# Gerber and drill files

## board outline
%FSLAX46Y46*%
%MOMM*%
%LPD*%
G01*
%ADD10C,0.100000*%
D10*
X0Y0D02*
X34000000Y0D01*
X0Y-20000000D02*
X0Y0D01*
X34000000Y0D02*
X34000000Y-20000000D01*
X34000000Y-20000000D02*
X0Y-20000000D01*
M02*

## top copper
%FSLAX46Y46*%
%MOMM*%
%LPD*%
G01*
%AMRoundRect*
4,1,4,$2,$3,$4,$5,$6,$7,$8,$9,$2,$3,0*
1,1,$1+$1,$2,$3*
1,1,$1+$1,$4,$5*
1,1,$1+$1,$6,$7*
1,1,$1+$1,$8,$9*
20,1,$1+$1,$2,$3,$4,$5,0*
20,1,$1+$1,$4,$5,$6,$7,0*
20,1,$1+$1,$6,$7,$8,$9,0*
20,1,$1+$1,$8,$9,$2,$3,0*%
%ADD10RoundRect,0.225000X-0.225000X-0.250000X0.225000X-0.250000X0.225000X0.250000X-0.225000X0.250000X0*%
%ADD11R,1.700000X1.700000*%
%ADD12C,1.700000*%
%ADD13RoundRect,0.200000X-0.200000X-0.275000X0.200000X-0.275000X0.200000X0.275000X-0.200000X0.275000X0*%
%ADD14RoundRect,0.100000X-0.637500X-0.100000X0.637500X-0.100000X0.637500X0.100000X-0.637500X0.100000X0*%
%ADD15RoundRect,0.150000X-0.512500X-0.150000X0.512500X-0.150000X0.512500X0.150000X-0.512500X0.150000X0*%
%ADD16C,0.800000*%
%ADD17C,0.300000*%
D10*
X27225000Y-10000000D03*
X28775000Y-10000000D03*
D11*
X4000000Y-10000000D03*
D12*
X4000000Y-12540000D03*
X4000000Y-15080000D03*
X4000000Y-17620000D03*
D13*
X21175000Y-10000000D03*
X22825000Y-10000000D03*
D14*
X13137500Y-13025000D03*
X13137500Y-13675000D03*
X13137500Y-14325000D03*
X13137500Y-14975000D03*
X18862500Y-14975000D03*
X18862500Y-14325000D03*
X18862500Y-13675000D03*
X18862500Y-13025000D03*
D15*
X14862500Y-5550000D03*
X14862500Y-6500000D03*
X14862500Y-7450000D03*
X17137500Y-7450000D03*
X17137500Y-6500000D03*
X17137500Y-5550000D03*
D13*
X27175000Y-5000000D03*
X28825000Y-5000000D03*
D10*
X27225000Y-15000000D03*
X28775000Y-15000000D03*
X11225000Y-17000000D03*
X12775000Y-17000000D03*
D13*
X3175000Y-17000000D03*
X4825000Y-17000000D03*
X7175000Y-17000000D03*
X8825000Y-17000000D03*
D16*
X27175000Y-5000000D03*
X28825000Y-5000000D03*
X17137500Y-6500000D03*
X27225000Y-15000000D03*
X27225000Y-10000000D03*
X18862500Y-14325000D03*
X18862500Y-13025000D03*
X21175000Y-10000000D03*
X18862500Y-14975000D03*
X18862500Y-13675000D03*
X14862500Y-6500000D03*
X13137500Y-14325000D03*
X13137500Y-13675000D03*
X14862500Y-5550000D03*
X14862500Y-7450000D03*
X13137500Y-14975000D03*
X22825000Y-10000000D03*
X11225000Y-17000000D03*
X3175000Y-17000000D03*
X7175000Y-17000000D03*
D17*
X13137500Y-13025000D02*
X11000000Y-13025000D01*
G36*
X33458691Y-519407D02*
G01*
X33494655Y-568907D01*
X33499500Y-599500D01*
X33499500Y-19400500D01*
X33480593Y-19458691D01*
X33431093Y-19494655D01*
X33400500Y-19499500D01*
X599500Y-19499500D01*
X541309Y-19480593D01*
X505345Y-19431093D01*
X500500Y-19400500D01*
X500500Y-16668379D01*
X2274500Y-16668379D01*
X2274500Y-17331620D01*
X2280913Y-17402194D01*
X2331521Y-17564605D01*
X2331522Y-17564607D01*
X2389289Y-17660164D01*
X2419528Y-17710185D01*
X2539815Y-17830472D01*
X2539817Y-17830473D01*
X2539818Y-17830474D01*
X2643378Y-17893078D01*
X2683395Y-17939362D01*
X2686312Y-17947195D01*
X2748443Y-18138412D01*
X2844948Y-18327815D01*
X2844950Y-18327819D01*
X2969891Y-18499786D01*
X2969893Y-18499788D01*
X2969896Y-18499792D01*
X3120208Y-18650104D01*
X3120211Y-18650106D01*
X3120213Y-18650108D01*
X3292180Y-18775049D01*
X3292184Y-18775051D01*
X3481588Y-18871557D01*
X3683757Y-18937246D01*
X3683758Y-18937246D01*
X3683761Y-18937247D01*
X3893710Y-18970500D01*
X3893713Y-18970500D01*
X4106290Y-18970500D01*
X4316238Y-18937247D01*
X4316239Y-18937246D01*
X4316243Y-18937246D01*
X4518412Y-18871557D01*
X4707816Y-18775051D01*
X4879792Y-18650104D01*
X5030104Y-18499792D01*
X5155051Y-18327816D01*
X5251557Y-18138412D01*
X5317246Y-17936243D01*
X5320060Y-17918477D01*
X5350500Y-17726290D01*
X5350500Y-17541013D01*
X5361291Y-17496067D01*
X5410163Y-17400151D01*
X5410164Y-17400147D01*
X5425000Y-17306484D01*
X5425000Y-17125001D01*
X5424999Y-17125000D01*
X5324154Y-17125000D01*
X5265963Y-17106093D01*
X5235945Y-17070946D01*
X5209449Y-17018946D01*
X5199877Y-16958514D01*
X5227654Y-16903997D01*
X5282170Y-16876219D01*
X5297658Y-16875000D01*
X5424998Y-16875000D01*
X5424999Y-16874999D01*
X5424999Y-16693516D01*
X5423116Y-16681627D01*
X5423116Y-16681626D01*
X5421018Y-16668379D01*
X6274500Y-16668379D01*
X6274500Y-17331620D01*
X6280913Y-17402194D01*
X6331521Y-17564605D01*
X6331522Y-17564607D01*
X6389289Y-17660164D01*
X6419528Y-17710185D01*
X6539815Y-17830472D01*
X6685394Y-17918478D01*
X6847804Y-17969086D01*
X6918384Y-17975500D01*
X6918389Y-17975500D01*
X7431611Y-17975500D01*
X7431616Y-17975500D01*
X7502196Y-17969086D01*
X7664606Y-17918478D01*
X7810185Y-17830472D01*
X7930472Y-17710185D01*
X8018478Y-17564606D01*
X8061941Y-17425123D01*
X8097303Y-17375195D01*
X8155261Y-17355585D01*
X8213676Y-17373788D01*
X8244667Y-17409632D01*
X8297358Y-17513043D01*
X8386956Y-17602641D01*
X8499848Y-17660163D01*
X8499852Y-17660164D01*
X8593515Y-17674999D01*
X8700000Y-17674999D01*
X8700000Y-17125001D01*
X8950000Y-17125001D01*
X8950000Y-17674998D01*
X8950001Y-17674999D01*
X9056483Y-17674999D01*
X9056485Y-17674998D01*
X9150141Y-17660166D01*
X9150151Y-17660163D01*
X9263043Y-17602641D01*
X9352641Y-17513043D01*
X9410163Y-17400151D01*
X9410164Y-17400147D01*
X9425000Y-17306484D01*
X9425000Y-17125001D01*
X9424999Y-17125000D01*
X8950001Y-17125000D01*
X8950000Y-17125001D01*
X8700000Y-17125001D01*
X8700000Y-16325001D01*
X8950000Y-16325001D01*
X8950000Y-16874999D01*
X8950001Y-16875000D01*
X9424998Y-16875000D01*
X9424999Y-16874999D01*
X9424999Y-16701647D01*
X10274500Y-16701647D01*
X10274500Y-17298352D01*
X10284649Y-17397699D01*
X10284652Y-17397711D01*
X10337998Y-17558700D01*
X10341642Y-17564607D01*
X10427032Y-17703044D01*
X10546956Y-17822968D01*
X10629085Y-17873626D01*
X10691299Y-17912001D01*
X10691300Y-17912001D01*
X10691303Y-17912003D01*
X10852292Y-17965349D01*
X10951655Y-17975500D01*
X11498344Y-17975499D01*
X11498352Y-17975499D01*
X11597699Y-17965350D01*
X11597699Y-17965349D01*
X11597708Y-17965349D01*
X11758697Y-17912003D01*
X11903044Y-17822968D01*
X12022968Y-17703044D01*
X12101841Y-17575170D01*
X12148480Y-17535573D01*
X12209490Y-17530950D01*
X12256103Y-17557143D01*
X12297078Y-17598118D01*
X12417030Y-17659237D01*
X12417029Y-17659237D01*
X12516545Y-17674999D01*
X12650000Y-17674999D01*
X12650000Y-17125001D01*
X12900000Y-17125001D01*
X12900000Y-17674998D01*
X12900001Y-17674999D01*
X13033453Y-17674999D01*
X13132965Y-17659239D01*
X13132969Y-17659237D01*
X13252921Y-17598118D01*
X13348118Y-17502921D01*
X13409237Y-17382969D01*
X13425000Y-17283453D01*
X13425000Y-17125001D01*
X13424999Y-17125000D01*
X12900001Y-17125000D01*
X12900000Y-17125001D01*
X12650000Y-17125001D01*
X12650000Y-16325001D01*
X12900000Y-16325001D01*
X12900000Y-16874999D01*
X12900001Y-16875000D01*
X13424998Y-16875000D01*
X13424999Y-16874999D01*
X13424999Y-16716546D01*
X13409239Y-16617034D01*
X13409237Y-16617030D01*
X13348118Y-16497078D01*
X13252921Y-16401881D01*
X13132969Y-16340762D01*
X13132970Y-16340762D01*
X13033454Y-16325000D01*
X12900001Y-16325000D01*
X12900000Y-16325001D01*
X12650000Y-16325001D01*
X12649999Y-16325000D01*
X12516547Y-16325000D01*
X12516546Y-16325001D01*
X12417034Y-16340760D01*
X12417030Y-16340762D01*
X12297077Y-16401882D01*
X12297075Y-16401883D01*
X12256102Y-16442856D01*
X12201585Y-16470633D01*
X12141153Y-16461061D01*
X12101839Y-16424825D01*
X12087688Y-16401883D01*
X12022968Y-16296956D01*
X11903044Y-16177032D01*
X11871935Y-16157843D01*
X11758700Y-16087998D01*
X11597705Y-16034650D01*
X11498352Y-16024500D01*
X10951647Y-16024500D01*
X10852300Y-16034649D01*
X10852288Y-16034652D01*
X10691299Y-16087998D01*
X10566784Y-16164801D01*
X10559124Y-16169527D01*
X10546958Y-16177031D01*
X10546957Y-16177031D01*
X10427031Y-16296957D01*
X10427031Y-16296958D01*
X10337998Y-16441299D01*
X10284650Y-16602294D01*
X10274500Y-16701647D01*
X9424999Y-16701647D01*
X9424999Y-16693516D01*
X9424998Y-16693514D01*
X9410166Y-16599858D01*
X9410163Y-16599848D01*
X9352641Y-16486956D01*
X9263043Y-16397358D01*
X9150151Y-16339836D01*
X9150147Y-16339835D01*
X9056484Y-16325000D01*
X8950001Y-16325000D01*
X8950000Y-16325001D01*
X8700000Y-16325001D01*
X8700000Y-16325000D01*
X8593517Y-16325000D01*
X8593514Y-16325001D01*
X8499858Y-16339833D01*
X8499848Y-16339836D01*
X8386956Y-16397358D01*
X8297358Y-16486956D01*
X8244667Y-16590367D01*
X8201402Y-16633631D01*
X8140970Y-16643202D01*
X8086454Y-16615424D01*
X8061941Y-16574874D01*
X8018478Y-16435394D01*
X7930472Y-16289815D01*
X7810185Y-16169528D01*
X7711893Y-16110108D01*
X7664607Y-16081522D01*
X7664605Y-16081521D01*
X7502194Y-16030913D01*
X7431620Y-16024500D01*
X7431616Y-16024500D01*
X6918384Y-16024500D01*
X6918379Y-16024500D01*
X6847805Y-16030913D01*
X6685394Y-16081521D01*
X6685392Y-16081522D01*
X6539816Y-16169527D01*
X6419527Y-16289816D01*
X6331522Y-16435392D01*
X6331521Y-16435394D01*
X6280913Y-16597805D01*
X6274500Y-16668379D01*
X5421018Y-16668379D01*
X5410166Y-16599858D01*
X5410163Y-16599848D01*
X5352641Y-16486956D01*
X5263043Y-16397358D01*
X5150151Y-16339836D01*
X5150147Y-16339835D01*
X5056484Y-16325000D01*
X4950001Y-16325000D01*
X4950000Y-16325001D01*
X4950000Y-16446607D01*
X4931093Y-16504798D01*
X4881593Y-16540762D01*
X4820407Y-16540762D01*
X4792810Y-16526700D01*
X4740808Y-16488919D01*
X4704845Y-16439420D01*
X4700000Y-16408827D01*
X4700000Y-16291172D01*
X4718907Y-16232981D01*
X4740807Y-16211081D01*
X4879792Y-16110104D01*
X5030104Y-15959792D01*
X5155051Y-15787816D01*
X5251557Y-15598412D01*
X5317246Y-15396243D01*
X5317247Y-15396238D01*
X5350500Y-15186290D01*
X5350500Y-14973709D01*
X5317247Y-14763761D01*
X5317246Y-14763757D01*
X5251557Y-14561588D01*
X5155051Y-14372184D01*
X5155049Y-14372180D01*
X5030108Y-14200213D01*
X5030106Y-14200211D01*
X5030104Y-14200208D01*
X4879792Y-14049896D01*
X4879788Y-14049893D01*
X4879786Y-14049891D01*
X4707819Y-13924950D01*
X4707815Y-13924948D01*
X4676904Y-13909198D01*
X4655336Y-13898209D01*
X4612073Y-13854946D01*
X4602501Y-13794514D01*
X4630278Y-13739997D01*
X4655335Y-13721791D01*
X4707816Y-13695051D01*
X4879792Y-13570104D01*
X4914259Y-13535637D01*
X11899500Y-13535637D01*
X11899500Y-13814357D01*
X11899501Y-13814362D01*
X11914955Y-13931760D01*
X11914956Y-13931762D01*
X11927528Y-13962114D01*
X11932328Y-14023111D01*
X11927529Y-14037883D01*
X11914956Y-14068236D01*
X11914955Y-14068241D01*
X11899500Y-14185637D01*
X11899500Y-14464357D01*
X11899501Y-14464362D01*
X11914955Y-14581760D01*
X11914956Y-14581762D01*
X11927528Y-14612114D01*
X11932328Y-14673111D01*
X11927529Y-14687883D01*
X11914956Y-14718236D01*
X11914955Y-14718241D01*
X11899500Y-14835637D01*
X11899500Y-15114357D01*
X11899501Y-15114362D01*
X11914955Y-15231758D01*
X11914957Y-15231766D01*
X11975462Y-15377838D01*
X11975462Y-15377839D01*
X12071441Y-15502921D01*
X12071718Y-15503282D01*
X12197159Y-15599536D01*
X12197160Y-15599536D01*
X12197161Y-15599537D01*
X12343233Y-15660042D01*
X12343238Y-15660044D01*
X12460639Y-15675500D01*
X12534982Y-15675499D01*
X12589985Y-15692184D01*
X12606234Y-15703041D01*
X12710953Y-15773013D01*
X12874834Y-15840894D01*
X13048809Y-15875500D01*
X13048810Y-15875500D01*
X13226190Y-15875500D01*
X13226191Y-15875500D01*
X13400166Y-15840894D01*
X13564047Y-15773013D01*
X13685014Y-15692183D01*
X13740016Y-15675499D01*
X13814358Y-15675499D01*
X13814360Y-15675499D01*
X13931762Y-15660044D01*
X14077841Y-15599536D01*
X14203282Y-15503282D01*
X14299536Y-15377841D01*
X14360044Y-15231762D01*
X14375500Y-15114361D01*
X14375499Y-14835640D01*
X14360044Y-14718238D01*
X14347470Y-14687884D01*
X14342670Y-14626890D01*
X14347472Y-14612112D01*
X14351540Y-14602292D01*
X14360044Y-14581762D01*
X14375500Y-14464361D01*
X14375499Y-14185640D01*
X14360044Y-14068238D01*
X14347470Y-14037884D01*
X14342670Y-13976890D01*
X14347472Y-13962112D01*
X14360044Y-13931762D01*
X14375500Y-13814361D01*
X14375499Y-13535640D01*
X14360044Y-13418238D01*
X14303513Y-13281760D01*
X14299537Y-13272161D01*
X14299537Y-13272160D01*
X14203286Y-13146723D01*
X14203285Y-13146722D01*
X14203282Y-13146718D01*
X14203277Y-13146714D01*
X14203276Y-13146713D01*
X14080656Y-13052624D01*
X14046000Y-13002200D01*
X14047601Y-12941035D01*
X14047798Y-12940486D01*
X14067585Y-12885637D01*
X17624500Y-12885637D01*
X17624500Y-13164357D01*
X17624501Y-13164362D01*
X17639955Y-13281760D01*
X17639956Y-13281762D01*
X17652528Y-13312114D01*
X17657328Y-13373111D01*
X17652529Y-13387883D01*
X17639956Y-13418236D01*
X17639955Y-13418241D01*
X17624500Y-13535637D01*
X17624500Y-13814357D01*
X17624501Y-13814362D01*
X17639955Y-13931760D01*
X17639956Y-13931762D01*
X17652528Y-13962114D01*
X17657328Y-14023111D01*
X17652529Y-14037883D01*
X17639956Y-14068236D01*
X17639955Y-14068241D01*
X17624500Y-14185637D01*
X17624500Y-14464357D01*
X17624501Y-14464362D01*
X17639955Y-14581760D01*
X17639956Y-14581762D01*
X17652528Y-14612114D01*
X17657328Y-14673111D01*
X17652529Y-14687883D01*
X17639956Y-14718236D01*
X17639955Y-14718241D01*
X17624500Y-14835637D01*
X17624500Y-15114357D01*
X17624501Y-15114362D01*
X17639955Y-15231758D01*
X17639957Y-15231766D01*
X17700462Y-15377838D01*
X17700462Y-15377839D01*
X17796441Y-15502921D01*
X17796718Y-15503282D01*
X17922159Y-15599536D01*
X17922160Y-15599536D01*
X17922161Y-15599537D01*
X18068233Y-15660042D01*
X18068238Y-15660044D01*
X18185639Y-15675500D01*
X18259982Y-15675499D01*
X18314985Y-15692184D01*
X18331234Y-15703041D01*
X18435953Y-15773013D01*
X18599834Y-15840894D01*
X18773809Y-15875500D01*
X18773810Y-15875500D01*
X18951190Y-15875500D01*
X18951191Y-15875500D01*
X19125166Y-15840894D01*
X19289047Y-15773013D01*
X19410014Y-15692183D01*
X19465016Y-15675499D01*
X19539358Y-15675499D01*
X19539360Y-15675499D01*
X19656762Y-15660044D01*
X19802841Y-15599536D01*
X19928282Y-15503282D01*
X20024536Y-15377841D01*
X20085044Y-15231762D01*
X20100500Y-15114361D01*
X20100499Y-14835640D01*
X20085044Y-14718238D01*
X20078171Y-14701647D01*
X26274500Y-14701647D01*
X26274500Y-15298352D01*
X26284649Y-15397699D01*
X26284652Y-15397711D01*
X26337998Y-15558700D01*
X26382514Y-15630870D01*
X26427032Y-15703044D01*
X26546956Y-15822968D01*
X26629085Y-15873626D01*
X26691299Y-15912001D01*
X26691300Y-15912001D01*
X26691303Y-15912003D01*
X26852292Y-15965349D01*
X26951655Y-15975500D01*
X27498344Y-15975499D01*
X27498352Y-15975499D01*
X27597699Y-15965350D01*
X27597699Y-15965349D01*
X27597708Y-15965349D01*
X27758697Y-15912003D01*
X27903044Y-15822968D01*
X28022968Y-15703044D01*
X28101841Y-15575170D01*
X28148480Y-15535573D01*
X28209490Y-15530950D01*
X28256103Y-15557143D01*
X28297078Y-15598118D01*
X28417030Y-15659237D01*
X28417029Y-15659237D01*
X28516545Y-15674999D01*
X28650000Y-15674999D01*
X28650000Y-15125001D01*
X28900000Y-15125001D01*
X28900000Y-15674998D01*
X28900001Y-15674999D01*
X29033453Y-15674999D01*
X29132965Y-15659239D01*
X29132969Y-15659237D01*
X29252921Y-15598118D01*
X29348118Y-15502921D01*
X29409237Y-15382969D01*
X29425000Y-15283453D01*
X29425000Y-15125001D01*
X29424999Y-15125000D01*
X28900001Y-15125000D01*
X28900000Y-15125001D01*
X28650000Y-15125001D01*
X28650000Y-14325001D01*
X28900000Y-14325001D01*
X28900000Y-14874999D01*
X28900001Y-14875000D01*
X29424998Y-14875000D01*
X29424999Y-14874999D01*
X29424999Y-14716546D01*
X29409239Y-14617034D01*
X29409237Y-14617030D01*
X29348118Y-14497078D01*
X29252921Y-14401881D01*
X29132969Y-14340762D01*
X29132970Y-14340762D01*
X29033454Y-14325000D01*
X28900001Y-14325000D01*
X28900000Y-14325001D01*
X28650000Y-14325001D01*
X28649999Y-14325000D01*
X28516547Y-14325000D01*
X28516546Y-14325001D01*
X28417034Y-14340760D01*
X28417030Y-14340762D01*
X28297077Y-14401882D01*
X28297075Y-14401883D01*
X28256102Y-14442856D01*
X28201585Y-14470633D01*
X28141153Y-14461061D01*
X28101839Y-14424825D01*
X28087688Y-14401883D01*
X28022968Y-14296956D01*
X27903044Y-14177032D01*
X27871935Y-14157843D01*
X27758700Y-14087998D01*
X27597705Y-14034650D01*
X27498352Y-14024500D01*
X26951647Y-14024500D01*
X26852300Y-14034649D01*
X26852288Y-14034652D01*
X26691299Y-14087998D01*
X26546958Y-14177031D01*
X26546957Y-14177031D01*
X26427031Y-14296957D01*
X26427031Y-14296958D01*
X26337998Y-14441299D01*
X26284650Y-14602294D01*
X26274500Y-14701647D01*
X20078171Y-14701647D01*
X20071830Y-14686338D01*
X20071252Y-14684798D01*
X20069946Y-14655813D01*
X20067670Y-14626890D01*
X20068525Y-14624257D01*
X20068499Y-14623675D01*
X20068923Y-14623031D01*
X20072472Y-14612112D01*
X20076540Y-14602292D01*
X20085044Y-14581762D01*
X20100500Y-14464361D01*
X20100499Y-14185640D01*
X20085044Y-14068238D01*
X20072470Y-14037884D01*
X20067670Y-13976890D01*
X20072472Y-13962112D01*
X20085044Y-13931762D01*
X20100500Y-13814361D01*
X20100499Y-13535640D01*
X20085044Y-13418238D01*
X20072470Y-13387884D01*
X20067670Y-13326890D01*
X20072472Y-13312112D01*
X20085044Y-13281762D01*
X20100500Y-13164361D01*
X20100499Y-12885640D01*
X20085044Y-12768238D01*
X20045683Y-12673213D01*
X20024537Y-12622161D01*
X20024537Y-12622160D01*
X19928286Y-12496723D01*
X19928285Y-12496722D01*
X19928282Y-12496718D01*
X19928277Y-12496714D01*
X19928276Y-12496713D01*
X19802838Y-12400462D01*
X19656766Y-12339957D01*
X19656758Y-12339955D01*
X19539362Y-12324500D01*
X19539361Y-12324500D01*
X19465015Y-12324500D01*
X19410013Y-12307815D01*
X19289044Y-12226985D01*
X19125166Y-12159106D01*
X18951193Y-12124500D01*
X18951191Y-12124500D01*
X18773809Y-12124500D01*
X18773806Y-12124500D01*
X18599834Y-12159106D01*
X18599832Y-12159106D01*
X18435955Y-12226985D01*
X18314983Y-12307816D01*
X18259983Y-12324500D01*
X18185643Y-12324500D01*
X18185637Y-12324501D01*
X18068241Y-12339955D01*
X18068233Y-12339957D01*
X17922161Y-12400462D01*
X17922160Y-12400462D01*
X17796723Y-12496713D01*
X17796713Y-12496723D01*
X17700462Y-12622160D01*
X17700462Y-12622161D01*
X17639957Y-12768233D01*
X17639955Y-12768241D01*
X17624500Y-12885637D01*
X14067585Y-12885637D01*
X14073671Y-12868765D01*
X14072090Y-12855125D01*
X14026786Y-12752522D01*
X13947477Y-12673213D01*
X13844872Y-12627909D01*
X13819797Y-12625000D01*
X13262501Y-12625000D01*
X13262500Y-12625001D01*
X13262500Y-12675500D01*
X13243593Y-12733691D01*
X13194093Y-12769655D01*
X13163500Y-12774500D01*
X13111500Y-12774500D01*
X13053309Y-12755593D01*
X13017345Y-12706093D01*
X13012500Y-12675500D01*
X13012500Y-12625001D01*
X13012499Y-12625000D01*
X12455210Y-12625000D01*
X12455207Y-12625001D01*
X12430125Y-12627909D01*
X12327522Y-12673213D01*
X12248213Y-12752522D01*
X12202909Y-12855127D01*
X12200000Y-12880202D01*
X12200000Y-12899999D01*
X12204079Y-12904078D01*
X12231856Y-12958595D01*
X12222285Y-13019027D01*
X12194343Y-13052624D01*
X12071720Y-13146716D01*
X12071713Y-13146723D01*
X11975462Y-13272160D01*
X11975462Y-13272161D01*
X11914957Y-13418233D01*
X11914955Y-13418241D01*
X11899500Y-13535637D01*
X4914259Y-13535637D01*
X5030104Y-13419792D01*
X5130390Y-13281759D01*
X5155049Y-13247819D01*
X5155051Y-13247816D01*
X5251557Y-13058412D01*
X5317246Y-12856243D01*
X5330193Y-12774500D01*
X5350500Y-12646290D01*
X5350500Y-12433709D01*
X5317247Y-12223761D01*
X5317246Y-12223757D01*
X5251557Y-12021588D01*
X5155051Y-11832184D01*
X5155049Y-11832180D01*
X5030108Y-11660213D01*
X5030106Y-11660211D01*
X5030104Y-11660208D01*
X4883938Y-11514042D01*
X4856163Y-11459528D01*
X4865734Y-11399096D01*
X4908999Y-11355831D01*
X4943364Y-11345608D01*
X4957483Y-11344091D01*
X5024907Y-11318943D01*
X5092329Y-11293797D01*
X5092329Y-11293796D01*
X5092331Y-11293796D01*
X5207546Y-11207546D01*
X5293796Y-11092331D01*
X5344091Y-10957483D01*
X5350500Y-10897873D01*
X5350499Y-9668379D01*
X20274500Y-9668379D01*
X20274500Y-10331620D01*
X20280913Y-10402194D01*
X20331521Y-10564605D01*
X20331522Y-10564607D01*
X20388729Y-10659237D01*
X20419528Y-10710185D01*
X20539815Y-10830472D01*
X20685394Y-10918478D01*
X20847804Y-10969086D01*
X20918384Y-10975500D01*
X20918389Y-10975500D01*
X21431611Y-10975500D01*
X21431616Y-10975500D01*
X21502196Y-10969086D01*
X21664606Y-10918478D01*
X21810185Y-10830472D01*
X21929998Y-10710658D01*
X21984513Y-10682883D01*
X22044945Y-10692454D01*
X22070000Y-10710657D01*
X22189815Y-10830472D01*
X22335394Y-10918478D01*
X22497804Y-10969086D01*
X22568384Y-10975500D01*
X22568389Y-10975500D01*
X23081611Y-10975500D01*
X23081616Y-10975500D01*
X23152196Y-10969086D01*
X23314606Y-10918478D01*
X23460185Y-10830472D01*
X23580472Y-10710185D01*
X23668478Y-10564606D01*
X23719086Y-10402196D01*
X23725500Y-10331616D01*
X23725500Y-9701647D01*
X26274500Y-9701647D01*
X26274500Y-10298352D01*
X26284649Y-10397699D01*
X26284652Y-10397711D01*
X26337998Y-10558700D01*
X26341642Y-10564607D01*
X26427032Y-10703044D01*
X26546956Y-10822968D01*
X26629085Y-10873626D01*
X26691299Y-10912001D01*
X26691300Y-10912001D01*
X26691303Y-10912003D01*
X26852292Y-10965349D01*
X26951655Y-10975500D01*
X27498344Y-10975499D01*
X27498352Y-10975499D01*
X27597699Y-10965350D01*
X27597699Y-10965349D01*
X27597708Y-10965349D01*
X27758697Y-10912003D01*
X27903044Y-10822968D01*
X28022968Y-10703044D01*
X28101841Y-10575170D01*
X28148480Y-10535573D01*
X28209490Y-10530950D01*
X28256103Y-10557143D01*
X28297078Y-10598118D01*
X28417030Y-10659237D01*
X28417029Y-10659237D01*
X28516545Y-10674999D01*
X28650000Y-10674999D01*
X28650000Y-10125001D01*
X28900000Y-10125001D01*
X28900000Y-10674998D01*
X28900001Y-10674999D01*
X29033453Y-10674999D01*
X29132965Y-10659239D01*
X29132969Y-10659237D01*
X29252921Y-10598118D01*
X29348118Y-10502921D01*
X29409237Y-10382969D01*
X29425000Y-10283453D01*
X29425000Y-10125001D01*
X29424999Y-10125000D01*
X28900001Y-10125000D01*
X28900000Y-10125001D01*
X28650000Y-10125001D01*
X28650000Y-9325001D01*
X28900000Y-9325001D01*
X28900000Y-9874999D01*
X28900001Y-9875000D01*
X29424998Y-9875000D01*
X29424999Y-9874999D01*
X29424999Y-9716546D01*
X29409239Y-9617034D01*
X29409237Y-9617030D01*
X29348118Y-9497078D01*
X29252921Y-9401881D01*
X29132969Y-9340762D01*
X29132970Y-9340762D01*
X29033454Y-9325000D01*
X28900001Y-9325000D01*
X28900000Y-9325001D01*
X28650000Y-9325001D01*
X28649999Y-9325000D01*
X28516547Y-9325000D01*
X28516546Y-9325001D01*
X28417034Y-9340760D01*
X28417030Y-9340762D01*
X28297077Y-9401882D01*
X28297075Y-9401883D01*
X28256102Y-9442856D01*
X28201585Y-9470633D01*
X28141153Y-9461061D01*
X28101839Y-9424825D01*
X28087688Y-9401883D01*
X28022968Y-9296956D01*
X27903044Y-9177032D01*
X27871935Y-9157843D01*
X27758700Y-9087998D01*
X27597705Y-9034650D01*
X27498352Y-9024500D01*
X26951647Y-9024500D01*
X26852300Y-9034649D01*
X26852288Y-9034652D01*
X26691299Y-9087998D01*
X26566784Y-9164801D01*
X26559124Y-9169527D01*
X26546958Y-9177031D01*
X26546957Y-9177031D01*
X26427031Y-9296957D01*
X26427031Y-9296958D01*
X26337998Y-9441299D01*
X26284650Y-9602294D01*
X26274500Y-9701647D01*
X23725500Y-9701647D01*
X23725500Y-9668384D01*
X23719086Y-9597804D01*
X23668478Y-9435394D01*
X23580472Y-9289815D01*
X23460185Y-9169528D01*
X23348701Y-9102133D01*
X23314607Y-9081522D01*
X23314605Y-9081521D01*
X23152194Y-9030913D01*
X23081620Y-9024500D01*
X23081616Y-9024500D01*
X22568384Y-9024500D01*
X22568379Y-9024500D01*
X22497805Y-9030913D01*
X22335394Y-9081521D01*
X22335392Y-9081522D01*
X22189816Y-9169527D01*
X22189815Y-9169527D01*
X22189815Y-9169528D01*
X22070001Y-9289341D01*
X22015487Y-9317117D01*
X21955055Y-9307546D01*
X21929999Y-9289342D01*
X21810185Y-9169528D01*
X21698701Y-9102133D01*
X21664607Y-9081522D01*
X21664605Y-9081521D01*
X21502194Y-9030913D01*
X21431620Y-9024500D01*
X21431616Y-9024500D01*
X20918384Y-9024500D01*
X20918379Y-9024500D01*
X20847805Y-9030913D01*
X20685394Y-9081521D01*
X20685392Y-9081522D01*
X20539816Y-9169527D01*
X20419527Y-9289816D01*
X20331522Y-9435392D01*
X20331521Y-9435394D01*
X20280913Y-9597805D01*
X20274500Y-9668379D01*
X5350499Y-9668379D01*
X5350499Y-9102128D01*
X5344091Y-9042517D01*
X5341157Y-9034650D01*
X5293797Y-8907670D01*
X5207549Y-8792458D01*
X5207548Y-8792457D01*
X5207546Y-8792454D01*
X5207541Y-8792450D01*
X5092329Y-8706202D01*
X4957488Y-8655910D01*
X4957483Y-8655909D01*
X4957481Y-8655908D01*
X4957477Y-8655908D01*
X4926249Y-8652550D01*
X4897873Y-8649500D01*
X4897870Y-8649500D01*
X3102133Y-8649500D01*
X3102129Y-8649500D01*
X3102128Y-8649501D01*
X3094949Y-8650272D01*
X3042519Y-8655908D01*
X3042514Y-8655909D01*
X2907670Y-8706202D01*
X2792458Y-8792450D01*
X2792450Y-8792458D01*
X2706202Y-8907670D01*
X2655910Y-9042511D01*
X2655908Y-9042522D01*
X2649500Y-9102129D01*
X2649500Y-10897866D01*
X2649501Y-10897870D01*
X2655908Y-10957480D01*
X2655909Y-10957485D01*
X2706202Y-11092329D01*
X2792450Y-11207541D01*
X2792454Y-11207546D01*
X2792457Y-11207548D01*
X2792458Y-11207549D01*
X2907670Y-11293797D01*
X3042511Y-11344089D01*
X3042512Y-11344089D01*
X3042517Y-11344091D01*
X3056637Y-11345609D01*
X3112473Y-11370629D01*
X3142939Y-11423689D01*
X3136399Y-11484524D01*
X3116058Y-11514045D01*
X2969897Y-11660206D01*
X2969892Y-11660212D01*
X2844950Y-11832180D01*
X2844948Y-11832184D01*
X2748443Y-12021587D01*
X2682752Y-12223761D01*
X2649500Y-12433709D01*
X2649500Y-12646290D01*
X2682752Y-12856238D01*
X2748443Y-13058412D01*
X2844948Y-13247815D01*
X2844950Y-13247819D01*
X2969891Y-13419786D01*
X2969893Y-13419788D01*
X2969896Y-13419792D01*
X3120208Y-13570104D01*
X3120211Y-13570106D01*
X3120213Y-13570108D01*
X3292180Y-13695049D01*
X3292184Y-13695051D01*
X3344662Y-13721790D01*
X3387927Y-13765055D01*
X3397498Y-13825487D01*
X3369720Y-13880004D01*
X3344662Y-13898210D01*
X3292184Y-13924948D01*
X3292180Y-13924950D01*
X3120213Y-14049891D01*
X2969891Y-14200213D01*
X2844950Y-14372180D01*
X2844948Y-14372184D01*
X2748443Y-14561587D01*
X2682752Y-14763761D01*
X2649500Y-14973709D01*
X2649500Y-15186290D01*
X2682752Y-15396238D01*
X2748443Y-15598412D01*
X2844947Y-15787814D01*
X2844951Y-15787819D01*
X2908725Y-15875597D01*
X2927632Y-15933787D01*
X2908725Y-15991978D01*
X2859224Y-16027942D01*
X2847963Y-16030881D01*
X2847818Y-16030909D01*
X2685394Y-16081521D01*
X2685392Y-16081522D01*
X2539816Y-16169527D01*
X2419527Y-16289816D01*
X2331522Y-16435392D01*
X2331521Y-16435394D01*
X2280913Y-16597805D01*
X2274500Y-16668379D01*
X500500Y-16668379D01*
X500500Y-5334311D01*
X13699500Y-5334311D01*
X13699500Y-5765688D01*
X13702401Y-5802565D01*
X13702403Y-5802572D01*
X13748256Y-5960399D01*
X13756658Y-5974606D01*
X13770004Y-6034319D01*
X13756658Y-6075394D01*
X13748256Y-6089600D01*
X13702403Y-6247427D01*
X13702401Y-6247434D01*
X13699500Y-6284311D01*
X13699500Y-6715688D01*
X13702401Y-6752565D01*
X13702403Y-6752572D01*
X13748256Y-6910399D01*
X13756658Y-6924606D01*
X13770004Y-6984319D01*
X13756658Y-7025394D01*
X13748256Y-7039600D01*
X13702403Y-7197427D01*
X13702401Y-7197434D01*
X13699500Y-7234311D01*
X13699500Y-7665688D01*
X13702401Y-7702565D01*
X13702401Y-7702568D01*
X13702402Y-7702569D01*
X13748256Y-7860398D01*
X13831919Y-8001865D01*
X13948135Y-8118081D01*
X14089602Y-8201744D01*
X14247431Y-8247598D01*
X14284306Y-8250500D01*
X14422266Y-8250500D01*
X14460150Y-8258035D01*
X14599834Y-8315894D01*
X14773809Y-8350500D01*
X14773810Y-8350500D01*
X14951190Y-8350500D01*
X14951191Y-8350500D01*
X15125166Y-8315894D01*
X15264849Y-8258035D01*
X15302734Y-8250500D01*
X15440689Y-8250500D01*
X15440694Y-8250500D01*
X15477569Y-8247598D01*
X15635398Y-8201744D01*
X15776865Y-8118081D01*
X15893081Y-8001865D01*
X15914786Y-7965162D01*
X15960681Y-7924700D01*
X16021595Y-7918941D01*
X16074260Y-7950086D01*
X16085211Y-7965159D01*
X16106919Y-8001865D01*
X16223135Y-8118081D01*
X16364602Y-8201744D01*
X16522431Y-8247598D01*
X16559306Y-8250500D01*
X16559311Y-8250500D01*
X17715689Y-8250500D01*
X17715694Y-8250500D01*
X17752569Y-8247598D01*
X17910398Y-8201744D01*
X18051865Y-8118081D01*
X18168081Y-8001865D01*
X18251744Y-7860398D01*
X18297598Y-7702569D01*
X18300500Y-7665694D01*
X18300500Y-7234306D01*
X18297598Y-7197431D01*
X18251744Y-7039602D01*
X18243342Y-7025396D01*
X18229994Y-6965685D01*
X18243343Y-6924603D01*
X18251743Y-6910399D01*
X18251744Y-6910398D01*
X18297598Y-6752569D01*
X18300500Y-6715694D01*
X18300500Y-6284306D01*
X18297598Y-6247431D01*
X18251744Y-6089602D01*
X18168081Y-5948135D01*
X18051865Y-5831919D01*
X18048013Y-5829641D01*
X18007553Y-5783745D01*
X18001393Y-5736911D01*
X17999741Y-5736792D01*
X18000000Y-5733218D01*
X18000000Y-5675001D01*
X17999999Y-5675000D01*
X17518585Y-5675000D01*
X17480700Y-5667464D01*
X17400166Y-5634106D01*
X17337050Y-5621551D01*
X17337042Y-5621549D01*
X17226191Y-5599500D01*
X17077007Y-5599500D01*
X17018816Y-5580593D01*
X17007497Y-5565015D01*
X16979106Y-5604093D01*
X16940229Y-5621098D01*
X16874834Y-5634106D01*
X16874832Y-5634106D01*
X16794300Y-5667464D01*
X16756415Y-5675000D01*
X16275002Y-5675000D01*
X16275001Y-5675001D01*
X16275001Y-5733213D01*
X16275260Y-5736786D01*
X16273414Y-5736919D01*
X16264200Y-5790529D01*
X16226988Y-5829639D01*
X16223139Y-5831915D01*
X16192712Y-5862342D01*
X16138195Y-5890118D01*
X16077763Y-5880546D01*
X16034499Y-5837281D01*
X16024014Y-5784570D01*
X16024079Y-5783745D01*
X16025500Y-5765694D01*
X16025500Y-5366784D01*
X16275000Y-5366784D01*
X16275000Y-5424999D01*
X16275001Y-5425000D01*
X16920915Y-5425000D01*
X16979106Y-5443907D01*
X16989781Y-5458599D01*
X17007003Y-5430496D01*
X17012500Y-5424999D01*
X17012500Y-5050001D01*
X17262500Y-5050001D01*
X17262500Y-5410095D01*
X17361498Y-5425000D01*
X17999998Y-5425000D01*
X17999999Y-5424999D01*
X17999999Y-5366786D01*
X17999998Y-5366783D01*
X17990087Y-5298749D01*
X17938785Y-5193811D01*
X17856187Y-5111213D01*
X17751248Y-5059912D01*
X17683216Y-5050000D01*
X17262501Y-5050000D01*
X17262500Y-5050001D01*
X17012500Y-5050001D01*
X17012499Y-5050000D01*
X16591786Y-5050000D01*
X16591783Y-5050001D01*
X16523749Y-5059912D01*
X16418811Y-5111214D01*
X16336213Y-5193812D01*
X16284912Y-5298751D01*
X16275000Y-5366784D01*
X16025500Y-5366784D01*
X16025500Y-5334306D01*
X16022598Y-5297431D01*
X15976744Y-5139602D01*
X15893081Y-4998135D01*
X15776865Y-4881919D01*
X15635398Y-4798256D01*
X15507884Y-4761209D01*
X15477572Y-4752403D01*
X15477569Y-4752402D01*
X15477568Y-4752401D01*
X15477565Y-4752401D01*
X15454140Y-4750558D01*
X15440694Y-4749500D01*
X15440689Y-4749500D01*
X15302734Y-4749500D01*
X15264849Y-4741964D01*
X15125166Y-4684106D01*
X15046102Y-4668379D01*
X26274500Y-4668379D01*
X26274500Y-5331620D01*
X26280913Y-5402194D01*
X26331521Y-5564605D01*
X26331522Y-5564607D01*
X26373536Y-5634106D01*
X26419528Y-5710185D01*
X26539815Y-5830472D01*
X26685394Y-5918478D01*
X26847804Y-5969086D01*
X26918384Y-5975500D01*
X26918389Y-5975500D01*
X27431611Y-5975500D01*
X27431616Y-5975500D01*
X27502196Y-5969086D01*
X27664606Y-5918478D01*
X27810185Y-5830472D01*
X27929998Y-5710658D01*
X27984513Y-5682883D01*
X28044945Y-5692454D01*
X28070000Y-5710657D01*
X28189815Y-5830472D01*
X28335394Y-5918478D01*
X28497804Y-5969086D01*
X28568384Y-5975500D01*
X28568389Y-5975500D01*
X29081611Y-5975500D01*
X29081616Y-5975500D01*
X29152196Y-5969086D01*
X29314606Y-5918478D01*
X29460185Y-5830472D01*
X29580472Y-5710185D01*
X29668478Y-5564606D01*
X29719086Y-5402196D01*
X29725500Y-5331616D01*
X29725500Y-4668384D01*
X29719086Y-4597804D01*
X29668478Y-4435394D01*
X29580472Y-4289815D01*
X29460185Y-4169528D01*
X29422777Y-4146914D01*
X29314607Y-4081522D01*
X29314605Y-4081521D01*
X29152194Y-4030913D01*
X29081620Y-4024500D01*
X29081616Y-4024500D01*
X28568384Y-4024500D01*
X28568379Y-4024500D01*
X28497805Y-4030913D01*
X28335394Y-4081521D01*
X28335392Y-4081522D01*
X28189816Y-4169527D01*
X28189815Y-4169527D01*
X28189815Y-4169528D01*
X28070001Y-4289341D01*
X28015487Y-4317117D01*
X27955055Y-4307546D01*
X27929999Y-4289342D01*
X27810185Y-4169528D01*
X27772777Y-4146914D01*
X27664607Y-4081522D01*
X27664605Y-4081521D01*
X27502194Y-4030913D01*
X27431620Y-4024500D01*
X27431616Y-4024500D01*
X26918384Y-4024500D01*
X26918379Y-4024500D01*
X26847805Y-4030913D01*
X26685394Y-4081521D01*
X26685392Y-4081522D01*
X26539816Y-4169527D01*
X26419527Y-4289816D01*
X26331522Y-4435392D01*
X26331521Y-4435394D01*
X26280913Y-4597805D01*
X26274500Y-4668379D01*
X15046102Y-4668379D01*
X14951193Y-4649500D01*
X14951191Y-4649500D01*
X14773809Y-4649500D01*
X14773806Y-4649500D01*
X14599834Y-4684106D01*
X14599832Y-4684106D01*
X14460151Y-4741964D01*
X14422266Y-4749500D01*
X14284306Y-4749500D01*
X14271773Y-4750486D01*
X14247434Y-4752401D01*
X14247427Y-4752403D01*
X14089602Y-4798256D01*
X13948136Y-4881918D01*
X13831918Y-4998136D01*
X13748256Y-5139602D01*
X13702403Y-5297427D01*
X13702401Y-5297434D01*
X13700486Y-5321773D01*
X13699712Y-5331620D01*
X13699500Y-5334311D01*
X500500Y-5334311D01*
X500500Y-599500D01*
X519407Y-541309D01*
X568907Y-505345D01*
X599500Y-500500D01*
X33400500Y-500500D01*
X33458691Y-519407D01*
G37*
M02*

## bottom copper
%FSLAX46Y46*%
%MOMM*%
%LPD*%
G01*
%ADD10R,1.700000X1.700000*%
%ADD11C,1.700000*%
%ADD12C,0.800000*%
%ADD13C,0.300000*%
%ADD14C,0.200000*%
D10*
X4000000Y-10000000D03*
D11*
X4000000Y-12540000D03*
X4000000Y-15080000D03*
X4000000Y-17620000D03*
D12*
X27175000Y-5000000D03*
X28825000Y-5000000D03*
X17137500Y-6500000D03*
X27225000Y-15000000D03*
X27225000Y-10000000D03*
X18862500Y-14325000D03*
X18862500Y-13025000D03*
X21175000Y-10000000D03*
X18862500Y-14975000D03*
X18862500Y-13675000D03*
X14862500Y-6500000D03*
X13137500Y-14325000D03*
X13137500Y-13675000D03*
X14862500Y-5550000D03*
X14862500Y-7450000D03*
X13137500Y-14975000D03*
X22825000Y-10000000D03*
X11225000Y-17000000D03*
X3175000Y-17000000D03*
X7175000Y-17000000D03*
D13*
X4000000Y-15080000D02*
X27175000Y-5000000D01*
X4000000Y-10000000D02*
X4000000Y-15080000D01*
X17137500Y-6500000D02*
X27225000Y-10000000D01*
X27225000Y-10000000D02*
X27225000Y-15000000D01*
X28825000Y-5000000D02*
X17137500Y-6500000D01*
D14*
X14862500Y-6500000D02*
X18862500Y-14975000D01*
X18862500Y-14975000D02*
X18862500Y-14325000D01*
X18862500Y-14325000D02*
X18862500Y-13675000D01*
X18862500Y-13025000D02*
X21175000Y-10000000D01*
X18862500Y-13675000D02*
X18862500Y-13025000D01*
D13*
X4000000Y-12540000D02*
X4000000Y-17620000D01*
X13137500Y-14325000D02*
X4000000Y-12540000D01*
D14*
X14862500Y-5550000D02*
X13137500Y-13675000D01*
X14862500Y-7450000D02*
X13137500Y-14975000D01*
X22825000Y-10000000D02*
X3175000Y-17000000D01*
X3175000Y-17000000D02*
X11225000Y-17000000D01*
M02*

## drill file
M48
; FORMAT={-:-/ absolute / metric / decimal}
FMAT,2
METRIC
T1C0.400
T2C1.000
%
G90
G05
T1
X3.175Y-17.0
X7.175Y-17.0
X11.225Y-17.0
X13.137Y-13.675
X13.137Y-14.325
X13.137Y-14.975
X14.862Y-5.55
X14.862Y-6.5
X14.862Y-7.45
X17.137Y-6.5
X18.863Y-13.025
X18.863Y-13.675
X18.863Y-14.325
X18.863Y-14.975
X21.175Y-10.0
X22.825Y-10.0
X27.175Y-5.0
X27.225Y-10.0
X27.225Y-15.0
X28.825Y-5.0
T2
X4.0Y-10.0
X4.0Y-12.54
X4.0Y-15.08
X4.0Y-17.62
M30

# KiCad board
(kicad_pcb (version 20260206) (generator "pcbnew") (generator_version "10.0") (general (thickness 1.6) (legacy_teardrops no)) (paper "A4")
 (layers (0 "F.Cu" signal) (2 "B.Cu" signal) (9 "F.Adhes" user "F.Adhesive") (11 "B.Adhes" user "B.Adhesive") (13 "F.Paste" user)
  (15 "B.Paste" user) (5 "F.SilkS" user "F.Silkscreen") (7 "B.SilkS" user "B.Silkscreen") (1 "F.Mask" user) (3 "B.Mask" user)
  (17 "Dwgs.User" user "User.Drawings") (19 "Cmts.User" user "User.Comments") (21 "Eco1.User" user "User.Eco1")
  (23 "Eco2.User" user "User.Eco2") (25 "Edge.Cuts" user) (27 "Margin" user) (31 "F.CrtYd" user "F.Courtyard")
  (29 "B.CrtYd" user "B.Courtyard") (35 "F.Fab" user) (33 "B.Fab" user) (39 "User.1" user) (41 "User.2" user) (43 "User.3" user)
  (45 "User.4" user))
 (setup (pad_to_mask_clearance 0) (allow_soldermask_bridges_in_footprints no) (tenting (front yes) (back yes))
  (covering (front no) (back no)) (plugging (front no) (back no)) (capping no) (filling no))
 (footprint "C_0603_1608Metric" (layer "F.Cu") (at 28 10)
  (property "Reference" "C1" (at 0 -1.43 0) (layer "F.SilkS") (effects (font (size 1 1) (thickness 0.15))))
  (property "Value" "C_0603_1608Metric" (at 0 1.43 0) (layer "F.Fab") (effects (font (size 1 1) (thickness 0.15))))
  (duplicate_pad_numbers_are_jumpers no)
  (pad "1" smd roundrect (at -0.775 0) (size 0.9 0.95) (layers "F.Cu" "F.Mask" "F.Paste") (roundrect_rratio 0.25) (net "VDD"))
  (pad "2" smd roundrect (at 0.775 0) (size 0.9 0.95) (layers "F.Cu" "F.Mask" "F.Paste") (roundrect_rratio 0.25) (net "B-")))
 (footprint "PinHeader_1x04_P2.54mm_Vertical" (layer "F.Cu") (at 4 10)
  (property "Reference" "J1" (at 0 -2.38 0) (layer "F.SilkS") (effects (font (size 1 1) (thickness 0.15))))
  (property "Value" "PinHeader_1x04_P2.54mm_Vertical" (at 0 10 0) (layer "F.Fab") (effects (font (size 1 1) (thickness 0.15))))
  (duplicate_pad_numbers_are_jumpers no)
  (pad "1" thru_hole rect (at 0 0) (size 1.7 1.7) (drill 1) (layers "*.Cu" "*.Mask") (remove_unused_layers no) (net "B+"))
  (pad "2" thru_hole circle (at 0 2.54) (size 1.7 1.7) (drill 1) (layers "*.Cu" "*.Mask") (remove_unused_layers no) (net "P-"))
  (pad "3" thru_hole circle (at 0 5.08) (size 1.7 1.7) (drill 1) (layers "*.Cu" "*.Mask") (remove_unused_layers no) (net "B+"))
  (pad "4" thru_hole circle (at 0 7.62) (size 1.7 1.7) (drill 1) (layers "*.Cu" "*.Mask") (remove_unused_layers no) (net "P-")))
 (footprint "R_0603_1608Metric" (layer "F.Cu") (at 22 10)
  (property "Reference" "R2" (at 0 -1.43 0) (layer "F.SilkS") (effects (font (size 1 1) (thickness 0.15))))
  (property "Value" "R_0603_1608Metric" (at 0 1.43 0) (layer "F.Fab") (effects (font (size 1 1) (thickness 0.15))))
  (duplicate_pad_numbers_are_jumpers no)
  (pad "1" smd roundrect (at -0.825 0) (size 0.8 0.95) (layers "F.Cu" "F.Mask" "F.Paste") (roundrect_rratio 0.25) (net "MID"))
  (pad "2" smd roundrect (at 0.825 0) (size 0.8 0.95) (layers "F.Cu" "F.Mask" "F.Paste") (roundrect_rratio 0.25) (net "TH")))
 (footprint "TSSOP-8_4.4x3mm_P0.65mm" (layer "F.Cu") (at 16 14)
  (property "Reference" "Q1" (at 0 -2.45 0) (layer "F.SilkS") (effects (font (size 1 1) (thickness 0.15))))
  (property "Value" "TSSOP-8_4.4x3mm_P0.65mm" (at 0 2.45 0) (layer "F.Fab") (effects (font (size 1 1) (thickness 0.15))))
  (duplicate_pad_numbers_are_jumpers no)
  (pad "1" smd roundrect (at -2.8625 -0.975) (size 1.475 0.4) (layers "F.Cu" "F.Mask" "F.Paste") (roundrect_rratio 0.25) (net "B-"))
  (pad "2" smd roundrect (at -2.8625 -0.325) (size 1.475 0.4) (layers "F.Cu" "F.Mask" "F.Paste") (roundrect_rratio 0.25) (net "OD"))
  (pad "3" smd roundrect (at -2.8625 0.325) (size 1.475 0.4) (layers "F.Cu" "F.Mask" "F.Paste") (roundrect_rratio 0.25) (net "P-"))
  (pad "4" smd roundrect (at -2.8625 0.975) (size 1.475 0.4) (layers "F.Cu" "F.Mask" "F.Paste") (roundrect_rratio 0.25) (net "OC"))
  (pad "5" smd roundrect (at 2.8625 0.975) (size 1.475 0.4) (layers "F.Cu" "F.Mask" "F.Paste") (roundrect_rratio 0.25) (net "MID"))
  (pad "6" smd roundrect (at 2.8625 0.325) (size 1.475 0.4) (layers "F.Cu" "F.Mask" "F.Paste") (roundrect_rratio 0.25) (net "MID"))
  (pad "7" smd roundrect (at 2.8625 -0.325) (size 1.475 0.4) (layers "F.Cu" "F.Mask" "F.Paste") (roundrect_rratio 0.25) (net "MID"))
  (pad "8" smd roundrect (at 2.8625 -0.975) (size 1.475 0.4) (layers "F.Cu" "F.Mask" "F.Paste") (roundrect_rratio 0.25) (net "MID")))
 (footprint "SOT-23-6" (layer "F.Cu") (at 16 6.5)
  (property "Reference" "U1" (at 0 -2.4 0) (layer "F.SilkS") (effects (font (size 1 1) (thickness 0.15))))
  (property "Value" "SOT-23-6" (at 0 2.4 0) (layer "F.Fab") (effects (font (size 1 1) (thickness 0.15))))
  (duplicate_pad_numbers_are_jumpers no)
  (pad "1" smd roundrect (at -1.1375 -0.95) (size 1.325 0.6) (layers "F.Cu" "F.Mask" "F.Paste") (roundrect_rratio 0.25) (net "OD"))
  (pad "2" smd roundrect (at -1.1375 0) (size 1.325 0.6) (layers "F.Cu" "F.Mask" "F.Paste") (roundrect_rratio 0.25) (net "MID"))
  (pad "3" smd roundrect (at -1.1375 0.95) (size 1.325 0.6) (layers "F.Cu" "F.Mask" "F.Paste") (roundrect_rratio 0.25) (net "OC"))
  (pad "4" smd roundrect (at 1.1375 0.95) (size 1.325 0.6) (layers "F.Cu" "F.Mask" "F.Paste") (roundrect_rratio 0.25))
  (pad "5" smd roundrect (at 1.1375 0) (size 1.325 0.6) (layers "F.Cu" "F.Mask" "F.Paste") (roundrect_rratio 0.25) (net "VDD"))
  (pad "6" smd roundrect (at 1.1375 -0.95) (size 1.325 0.6) (layers "F.Cu" "F.Mask" "F.Paste") (roundrect_rratio 0.25) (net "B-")))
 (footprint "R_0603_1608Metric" (layer "F.Cu") (at 28 5)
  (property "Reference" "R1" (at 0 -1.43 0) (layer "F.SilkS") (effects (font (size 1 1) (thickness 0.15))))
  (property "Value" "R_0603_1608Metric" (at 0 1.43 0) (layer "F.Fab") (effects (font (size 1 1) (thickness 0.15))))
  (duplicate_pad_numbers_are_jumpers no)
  (pad "1" smd roundrect (at -0.825 0) (size 0.8 0.95) (layers "F.Cu" "F.Mask" "F.Paste") (roundrect_rratio 0.25) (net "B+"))
  (pad "2" smd roundrect (at 0.825 0) (size 0.8 0.95) (layers "F.Cu" "F.Mask" "F.Paste") (roundrect_rratio 0.25) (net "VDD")))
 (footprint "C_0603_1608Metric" (layer "F.Cu") (at 28 15)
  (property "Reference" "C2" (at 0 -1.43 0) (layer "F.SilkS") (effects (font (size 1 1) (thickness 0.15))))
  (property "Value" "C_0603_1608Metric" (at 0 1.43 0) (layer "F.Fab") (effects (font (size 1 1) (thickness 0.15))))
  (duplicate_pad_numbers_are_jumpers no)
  (pad "1" smd roundrect (at -0.775 0) (size 0.9 0.95) (layers "F.Cu" "F.Mask" "F.Paste") (roundrect_rratio 0.25) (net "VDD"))
  (pad "2" smd roundrect (at 0.775 0) (size 0.9 0.95) (layers "F.Cu" "F.Mask" "F.Paste") (roundrect_rratio 0.25) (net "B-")))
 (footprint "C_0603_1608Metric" (layer "F.Cu") (at 12 17)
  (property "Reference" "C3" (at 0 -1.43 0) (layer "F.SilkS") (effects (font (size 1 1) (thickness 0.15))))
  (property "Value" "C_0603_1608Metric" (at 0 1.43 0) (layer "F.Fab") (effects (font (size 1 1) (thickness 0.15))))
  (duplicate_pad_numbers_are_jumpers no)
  (pad "1" smd roundrect (at -0.775 0) (size 0.9 0.95) (layers "F.Cu" "F.Mask" "F.Paste") (roundrect_rratio 0.25) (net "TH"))
  (pad "2" smd roundrect (at 0.775 0) (size 0.9 0.95) (layers "F.Cu" "F.Mask" "F.Paste") (roundrect_rratio 0.25) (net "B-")))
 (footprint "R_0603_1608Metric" (layer "F.Cu") (at 4 17)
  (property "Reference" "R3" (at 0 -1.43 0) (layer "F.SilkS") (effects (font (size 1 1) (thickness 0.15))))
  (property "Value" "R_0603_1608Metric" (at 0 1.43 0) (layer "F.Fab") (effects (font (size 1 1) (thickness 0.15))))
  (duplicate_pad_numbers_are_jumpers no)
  (pad "1" smd roundrect (at -0.825 0) (size 0.8 0.95) (layers "F.Cu" "F.Mask" "F.Paste") (roundrect_rratio 0.25) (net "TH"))
  (pad "2" smd roundrect (at 0.825 0) (size 0.8 0.95) (layers "F.Cu" "F.Mask" "F.Paste") (roundrect_rratio 0.25) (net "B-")))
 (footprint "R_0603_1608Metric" (layer "F.Cu") (at 8 17)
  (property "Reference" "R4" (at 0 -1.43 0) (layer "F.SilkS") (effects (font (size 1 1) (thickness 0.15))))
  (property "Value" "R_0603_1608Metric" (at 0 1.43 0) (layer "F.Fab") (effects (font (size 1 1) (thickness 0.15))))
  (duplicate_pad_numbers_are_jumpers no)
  (pad "1" smd roundrect (at -0.825 0) (size 0.8 0.95) (layers "F.Cu" "F.Mask" "F.Paste") (roundrect_rratio 0.25) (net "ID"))
  (pad "2" smd roundrect (at 0.825 0) (size 0.8 0.95) (layers "F.Cu" "F.Mask" "F.Paste") (roundrect_rratio 0.25) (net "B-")))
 (gr_line (start 0 0) (end 34 0) (stroke (width 0.1) (type default)) (layer "Edge.Cuts"))
 (gr_line (start 0 20) (end 0 0) (stroke (width 0.1) (type default)) (layer "Edge.Cuts"))
 (gr_line (start 34 0) (end 34 20) (stroke (width 0.1) (type default)) (layer "Edge.Cuts"))
 (gr_line (start 34 20) (end 0 20) (stroke (width 0.1) (type default)) (layer "Edge.Cuts"))
 (via (at 27.175 5) (size 0.8) (drill 0.4) (layers "F.Cu" "B.Cu") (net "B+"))
 (segment (start 4 15.08) (end 27.175 5) (width 0.3) (layer "B.Cu") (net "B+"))
 (segment (start 4 10) (end 4 15.08) (width 0.3) (layer "B.Cu") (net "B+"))
 (via (at 28.825 5) (size 0.8) (drill 0.4) (layers "F.Cu" "B.Cu") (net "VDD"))
 (via (at 17.1375 6.5) (size 0.8) (drill 0.4) (layers "F.Cu" "B.Cu") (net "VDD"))
 (via (at 27.225 15) (size 0.8) (drill 0.4) (layers "F.Cu" "B.Cu") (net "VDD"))
 (via (at 27.225 10) (size 0.8) (drill 0.4) (layers "F.Cu" "B.Cu") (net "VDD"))
 (segment (start 17.1375 6.5) (end 27.225 10) (width 0.3) (layer "B.Cu") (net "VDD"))
 (segment (start 27.225 10) (end 27.225 15) (width 0.3) (layer "B.Cu") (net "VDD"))
 (segment (start 28.825 5) (end 17.1375 6.5) (width 0.3) (layer "B.Cu") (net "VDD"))
 (segment (start 13.1375 13.025) (end 11 13.025) (width 0.3) (layer "F.Cu") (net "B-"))
 (via (at 18.8625 14.325) (size 0.8) (drill 0.4) (layers "F.Cu" "B.Cu") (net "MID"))
 (via (at 18.8625 13.025) (size 0.8) (drill 0.4) (layers "F.Cu" "B.Cu") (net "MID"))
 (via (at 21.175 10) (size 0.8) (drill 0.4) (layers "F.Cu" "B.Cu") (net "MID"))
 (via (at 18.8625 14.975) (size 0.8) (drill 0.4) (layers "F.Cu" "B.Cu") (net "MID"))
 (via (at 18.8625 13.675) (size 0.8) (drill 0.4) (layers "F.Cu" "B.Cu") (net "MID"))
 (via (at 14.8625 6.5) (size 0.8) (drill 0.4) (layers "F.Cu" "B.Cu") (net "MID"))
 (segment (start 14.8625 6.5) (end 18.8625 14.975) (width 0.2) (layer "B.Cu") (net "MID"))
 (segment (start 18.8625 14.975) (end 18.8625 14.325) (width 0.2) (layer "B.Cu") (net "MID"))
 (segment (start 18.8625 14.325) (end 18.8625 13.675) (width 0.2) (layer "B.Cu") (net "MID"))
 (segment (start 18.8625 13.025) (end 21.175 10) (width 0.2) (layer "B.Cu") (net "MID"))
 (segment (start 18.8625 13.675) (end 18.8625 13.025) (width 0.2) (layer "B.Cu") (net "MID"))
 (via (at 13.1375 14.325) (size 0.8) (drill 0.4) (layers "F.Cu" "B.Cu") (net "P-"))
 (segment (start 4 12.54) (end 4 17.62) (width 0.3) (layer "B.Cu") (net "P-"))
 (segment (start 13.1375 14.325) (end 4 12.54) (width 0.3) (layer "B.Cu") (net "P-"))
 (via (at 13.1375 13.675) (size 0.8) (drill 0.4) (layers "F.Cu" "B.Cu") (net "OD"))
 (via (at 14.8625 5.55) (size 0.8) (drill 0.4) (layers "F.Cu" "B.Cu") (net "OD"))
 (segment (start 14.8625 5.55) (end 13.1375 13.675) (width 0.2) (layer "B.Cu") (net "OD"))
 (via (at 14.8625 7.45) (size 0.8) (drill 0.4) (layers "F.Cu" "B.Cu") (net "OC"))
 (via (at 13.1375 14.975) (size 0.8) (drill 0.4) (layers "F.Cu" "B.Cu") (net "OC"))
 (segment (start 14.8625 7.45) (end 13.1375 14.975) (width 0.2) (layer "B.Cu") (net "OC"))
 (via (at 22.825 10) (size 0.8) (drill 0.4) (layers "F.Cu" "B.Cu") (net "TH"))
 (via (at 11.225 17) (size 0.8) (drill 0.4) (layers "F.Cu" "B.Cu") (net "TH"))
 (via (at 3.175 17) (size 0.8) (drill 0.4) (layers "F.Cu" "B.Cu") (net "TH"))
 (segment (start 22.825 10) (end 3.175 17) (width 0.2) (layer "B.Cu") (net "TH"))
 (segment (start 3.175 17) (end 11.225 17) (width 0.2) (layer "B.Cu") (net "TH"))
 (via (at 7.175 17) (size 0.8) (drill 0.4) (layers "F.Cu" "B.Cu") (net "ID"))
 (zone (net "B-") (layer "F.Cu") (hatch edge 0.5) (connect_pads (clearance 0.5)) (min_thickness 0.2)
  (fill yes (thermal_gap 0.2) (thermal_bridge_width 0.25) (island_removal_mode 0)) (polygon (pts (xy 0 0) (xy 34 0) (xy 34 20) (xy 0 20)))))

